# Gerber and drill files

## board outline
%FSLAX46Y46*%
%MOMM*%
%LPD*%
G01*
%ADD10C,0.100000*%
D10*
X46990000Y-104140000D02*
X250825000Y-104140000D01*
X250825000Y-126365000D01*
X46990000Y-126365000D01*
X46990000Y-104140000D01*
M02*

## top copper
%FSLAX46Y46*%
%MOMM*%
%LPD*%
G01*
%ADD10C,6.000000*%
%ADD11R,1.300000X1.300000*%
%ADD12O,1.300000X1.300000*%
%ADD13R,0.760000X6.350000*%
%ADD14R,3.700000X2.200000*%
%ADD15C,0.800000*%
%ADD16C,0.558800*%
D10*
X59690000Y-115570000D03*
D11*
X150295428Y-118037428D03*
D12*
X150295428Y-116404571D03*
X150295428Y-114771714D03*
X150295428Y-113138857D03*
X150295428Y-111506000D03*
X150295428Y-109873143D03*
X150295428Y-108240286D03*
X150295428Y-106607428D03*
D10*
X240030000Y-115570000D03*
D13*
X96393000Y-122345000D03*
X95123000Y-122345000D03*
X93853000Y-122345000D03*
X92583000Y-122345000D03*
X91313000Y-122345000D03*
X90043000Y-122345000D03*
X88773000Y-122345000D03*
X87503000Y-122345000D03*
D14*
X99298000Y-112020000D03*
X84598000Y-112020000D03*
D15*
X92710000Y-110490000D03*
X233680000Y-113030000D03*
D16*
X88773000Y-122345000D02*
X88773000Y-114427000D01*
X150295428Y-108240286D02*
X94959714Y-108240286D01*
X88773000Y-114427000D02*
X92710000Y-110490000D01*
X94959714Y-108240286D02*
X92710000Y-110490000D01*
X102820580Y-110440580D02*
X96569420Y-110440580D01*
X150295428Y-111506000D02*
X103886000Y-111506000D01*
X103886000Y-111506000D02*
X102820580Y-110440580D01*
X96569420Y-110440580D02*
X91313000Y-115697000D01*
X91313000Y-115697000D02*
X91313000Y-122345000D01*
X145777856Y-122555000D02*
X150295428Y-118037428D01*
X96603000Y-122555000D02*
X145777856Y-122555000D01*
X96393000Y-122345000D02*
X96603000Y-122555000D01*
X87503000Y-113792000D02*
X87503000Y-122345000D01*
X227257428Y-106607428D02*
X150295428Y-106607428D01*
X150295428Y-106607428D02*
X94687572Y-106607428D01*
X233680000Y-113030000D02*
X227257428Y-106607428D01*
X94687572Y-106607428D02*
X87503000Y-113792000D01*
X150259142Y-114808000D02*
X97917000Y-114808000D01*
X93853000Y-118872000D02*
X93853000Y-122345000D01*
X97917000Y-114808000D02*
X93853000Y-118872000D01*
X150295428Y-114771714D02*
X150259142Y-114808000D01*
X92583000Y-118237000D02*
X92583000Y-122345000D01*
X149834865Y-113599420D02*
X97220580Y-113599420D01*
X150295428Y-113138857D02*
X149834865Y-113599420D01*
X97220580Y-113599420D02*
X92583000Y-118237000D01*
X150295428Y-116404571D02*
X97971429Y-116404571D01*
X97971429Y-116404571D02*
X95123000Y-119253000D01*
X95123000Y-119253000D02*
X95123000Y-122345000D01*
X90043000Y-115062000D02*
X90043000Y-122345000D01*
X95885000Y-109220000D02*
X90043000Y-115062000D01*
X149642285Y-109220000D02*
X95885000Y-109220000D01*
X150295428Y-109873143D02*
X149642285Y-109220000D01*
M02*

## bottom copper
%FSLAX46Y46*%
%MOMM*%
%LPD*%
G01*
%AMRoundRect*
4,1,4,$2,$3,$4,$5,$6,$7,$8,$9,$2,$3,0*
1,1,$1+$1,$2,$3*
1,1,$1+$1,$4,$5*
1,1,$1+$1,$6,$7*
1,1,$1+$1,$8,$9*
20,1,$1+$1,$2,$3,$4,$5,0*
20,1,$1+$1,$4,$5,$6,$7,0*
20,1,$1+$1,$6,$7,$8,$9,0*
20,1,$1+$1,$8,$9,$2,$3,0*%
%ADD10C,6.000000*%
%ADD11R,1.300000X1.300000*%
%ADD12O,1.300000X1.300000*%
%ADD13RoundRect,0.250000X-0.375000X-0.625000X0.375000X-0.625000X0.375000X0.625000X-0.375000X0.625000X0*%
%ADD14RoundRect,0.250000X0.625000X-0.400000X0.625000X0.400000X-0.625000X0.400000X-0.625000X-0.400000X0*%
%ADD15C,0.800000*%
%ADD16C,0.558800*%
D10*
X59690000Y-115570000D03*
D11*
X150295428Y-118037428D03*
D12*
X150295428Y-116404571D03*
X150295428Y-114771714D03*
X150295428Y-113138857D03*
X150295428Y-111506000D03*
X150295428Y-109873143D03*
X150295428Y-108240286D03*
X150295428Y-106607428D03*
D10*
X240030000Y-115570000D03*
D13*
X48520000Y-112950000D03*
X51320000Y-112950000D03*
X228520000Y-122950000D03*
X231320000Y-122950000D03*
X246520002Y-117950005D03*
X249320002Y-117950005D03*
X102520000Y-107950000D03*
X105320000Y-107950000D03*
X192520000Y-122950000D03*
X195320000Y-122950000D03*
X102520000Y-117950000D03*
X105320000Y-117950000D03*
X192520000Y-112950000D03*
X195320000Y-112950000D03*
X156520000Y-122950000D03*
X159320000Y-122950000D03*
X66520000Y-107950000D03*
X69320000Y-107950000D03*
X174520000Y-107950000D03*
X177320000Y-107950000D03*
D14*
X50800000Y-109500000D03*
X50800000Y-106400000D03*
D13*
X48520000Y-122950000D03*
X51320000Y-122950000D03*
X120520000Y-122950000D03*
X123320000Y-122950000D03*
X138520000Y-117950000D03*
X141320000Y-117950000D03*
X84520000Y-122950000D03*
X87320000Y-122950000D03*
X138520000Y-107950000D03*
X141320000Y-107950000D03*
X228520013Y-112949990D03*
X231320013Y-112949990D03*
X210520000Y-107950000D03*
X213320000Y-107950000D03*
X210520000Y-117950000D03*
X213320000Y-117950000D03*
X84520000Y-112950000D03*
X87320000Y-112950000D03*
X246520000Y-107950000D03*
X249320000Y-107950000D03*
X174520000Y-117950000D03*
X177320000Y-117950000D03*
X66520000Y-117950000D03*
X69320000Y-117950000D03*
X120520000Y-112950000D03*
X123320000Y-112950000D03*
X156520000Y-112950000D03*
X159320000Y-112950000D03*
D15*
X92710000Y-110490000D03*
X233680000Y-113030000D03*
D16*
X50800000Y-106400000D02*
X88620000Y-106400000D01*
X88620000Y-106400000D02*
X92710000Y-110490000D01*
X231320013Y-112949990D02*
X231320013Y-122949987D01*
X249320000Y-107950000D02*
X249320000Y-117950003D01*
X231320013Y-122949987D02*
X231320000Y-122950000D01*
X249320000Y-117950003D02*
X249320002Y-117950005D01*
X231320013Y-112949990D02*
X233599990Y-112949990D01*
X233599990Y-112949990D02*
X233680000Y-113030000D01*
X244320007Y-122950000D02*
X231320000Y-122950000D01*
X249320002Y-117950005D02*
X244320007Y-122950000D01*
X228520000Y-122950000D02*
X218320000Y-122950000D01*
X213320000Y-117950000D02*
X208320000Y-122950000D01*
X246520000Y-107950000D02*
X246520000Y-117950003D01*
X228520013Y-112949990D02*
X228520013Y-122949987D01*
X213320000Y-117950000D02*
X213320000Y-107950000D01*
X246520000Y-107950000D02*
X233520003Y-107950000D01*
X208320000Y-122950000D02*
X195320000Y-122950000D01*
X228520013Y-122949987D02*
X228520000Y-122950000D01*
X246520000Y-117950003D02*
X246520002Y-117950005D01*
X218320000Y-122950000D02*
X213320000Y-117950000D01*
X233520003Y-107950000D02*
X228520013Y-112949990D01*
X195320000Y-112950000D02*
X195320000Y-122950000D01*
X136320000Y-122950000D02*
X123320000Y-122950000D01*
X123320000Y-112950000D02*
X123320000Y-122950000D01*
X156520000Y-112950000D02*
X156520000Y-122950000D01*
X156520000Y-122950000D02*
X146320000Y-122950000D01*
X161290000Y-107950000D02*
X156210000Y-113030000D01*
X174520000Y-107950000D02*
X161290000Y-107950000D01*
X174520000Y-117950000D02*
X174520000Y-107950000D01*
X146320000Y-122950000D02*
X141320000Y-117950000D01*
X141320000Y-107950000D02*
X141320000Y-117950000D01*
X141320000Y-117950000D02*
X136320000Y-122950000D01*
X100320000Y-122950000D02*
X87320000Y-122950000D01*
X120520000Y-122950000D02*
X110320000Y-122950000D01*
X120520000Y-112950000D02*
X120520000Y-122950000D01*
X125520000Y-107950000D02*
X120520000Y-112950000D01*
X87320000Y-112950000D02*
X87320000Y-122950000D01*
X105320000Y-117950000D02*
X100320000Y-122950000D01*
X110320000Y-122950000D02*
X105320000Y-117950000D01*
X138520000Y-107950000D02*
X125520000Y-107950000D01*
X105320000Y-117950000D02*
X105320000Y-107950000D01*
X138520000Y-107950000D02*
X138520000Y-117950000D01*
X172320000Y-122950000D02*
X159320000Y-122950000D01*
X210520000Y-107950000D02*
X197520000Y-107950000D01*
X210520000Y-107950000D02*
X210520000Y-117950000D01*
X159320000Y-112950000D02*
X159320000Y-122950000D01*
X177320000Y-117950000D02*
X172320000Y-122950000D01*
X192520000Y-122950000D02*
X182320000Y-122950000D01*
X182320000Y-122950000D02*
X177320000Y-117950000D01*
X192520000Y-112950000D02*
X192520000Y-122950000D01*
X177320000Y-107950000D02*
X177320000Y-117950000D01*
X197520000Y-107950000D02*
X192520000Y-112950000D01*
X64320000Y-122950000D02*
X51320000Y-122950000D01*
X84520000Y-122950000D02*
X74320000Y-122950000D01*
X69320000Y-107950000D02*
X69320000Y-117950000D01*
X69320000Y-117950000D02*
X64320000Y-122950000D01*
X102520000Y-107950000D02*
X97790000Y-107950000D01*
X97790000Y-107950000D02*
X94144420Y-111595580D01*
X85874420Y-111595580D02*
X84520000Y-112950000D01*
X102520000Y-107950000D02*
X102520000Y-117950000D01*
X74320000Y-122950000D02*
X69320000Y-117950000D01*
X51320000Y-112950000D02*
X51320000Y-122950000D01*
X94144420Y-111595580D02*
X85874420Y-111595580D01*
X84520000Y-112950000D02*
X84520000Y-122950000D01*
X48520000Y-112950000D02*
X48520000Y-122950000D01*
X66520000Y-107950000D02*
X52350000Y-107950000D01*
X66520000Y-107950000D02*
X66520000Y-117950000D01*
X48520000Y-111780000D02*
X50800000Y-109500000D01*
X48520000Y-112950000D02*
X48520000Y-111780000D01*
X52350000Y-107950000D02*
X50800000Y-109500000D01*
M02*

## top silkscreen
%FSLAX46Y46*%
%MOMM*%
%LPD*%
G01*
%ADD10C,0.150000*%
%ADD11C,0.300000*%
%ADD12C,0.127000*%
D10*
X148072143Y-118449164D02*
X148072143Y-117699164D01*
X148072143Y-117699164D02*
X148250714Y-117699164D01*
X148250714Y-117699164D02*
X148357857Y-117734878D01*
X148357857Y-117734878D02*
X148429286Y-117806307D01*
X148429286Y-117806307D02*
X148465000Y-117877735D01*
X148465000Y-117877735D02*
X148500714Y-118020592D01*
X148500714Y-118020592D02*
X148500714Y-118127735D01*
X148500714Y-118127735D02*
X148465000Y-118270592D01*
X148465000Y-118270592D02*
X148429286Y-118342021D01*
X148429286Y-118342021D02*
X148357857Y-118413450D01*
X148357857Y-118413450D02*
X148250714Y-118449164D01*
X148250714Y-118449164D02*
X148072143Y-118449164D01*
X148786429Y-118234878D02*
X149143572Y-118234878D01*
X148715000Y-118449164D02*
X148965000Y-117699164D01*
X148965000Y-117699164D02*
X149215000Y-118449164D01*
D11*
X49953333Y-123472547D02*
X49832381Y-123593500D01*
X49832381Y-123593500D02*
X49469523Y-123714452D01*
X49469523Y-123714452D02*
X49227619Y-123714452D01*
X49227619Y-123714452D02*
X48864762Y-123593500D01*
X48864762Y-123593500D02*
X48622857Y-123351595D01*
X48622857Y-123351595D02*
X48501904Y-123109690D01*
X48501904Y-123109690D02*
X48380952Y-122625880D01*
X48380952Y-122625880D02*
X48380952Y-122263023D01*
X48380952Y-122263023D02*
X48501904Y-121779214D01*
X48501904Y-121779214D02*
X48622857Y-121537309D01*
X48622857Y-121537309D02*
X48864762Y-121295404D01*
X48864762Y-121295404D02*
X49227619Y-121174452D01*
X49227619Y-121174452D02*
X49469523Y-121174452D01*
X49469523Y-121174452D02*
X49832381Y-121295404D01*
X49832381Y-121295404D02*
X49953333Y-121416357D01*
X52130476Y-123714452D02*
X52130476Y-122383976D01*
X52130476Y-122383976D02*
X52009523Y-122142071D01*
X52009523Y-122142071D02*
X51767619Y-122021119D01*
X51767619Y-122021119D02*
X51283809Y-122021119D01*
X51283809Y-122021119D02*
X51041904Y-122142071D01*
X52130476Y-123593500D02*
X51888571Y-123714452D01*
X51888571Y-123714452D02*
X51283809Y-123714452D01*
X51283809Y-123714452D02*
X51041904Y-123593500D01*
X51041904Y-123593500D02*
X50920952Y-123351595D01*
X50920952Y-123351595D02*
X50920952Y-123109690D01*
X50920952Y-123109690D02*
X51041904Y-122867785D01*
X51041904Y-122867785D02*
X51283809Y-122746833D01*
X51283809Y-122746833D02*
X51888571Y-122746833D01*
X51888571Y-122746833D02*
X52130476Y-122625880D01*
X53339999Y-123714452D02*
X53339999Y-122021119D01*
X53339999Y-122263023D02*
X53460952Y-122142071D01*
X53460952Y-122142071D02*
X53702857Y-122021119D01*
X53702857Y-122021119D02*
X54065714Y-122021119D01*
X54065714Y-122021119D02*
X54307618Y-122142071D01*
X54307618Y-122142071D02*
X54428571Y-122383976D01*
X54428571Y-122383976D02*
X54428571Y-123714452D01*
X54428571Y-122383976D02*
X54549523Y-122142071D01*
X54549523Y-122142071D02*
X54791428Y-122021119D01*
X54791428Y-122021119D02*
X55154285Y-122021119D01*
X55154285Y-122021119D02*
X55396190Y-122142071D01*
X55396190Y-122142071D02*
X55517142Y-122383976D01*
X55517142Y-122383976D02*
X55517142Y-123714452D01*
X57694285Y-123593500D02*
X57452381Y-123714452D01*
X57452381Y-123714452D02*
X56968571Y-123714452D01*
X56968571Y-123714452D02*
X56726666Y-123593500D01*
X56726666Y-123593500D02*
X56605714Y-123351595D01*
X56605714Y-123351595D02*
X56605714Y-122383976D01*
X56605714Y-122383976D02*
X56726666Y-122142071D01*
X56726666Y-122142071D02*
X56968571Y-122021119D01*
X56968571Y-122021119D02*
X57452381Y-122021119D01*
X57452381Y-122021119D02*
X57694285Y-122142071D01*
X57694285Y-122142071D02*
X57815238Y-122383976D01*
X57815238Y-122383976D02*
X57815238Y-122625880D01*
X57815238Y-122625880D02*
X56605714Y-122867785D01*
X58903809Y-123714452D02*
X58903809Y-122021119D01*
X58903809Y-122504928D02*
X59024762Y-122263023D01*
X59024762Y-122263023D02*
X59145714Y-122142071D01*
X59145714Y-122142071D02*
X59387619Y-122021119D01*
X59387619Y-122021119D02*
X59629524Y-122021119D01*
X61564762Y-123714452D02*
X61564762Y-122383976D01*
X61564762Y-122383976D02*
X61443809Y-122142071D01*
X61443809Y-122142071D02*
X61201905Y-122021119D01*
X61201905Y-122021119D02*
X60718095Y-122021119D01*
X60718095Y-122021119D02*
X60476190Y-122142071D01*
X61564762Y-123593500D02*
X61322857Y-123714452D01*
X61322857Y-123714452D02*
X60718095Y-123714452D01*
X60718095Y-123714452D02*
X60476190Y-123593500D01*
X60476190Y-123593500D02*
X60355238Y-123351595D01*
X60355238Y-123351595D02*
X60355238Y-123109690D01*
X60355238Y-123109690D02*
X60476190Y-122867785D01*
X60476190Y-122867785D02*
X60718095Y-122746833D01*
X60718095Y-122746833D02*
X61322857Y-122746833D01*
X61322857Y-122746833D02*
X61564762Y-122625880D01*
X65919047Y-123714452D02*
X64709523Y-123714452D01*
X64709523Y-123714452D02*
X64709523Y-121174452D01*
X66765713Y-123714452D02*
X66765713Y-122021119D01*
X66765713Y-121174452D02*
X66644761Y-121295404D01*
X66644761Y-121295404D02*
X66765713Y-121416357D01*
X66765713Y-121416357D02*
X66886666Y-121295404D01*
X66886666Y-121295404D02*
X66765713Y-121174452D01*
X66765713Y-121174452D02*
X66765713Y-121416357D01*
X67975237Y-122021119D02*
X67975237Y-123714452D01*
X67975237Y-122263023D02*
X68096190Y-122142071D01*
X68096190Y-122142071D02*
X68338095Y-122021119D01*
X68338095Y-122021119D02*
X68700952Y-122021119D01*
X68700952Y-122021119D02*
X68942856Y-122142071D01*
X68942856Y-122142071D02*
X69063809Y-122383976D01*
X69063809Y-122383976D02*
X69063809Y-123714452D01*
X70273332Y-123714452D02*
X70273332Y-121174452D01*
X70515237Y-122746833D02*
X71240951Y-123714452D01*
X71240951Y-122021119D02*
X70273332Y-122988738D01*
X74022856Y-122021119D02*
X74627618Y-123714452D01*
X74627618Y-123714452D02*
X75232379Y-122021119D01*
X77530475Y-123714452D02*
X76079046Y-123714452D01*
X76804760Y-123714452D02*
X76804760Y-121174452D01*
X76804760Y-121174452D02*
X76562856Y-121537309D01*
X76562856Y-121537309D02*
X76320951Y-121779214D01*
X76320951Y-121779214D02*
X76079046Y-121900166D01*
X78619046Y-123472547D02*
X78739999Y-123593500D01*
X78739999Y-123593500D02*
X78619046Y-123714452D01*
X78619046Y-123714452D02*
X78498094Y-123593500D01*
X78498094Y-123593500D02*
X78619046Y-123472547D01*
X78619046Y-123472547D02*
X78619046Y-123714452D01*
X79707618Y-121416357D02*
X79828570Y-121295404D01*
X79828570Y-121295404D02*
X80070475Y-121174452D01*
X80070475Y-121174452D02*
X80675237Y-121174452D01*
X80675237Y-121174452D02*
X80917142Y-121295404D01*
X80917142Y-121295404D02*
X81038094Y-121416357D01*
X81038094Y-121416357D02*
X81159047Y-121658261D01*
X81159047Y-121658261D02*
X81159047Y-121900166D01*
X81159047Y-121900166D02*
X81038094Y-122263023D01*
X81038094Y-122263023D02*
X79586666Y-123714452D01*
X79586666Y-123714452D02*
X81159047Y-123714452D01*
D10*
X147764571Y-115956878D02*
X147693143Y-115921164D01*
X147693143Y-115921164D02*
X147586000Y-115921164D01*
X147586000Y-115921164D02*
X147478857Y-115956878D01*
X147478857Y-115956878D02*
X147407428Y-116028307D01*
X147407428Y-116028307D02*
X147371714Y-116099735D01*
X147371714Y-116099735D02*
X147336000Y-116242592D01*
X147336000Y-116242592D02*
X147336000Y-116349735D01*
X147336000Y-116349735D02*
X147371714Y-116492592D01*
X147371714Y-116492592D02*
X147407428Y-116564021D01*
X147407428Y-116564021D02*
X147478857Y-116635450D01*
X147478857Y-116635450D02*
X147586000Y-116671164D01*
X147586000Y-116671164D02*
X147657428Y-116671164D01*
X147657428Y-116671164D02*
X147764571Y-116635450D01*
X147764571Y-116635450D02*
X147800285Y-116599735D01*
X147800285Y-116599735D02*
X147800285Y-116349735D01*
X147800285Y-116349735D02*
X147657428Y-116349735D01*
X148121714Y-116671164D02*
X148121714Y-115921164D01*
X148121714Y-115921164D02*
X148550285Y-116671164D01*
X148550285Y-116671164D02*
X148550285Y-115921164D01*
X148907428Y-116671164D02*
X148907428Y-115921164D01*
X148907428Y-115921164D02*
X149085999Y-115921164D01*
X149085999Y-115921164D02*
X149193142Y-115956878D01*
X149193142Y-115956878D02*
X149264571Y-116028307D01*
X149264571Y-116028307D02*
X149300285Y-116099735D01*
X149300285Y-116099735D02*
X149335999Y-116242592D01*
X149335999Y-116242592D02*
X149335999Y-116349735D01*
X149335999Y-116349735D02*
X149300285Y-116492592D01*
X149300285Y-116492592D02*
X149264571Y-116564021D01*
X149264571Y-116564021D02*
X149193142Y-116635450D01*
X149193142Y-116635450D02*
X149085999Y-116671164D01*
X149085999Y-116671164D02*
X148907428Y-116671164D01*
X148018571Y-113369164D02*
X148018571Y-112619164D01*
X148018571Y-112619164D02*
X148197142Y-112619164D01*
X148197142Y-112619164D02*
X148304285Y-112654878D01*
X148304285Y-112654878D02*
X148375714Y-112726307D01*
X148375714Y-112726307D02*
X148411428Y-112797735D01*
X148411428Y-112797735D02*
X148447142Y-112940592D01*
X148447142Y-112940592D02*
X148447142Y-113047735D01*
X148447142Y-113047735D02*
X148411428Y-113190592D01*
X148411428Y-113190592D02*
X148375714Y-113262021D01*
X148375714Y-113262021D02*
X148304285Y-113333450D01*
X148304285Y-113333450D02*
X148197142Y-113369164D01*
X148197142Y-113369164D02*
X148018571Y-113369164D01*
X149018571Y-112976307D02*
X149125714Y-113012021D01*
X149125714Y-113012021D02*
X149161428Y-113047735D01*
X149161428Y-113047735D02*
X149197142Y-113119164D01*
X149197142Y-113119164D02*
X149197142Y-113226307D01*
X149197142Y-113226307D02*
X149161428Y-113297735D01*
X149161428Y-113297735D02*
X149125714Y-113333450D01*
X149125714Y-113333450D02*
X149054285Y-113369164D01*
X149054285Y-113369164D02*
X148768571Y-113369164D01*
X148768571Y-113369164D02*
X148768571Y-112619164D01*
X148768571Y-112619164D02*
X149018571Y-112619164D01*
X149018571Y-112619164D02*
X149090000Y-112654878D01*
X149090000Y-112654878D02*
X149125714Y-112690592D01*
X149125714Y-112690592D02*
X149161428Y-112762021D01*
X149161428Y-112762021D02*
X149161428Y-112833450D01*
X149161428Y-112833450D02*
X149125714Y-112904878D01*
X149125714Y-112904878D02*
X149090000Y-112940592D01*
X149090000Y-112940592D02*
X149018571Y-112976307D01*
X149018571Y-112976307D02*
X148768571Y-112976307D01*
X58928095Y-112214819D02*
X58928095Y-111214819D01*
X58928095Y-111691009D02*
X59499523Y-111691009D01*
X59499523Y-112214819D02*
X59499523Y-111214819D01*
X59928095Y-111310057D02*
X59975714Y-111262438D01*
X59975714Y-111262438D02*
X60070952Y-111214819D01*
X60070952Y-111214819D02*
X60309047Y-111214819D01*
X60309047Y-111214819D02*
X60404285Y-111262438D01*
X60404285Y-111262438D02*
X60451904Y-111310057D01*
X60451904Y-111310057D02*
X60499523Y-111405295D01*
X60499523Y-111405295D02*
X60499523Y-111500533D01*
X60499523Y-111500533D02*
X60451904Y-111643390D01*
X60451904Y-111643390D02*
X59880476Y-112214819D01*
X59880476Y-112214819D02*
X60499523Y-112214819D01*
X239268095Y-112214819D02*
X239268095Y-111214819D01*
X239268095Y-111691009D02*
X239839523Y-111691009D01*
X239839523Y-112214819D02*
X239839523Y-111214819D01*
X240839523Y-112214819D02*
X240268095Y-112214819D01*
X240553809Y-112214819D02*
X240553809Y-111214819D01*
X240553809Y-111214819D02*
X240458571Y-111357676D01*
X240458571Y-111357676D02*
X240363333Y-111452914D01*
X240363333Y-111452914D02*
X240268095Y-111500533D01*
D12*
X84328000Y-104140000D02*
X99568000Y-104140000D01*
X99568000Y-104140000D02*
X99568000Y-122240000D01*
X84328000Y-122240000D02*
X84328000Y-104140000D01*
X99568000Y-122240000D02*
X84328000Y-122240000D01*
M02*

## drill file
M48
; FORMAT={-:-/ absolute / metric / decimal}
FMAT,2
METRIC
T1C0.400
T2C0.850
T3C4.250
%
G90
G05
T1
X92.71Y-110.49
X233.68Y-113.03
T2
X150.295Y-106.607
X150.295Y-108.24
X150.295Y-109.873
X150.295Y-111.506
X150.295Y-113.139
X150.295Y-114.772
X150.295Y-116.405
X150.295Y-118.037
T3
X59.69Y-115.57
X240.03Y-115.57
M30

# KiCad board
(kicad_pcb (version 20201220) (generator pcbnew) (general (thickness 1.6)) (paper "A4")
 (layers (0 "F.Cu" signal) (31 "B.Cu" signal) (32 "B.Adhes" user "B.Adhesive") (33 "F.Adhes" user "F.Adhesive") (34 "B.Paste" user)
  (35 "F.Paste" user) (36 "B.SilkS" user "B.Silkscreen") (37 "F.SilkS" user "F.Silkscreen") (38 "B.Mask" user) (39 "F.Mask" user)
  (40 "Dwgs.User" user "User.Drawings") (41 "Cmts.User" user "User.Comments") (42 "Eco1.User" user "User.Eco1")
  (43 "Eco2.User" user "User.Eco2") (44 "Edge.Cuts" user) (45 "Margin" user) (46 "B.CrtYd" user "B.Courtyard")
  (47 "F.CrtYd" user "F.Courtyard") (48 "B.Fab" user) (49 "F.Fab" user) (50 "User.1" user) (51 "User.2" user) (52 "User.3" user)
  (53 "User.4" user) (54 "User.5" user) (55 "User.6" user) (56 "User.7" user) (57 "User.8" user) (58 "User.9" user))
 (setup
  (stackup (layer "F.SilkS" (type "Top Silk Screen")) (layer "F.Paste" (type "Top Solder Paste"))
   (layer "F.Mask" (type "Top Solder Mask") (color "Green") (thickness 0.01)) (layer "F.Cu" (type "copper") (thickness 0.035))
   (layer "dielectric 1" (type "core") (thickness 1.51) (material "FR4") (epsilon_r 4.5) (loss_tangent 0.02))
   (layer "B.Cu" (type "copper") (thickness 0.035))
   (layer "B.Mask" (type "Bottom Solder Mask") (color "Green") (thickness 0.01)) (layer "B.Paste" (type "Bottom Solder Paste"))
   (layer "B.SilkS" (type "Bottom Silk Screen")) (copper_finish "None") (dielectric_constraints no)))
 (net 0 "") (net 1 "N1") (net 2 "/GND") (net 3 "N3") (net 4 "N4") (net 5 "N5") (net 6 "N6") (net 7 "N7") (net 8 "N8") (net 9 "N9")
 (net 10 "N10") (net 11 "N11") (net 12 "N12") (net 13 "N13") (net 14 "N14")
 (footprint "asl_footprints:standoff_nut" (layer "F.Cu") (at 59.69 115.57)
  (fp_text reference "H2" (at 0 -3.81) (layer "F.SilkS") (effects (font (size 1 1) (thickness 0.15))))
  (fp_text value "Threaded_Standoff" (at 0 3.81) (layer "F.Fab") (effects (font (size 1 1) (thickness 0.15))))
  (pad "M3" thru_hole circle (at 0 0) (size 6 6) (drill 4.25) (layers *.Cu *.Mask)))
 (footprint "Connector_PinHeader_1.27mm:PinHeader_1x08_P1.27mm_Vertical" (layer "F.Cu") (at 150.295428 112.322429 180)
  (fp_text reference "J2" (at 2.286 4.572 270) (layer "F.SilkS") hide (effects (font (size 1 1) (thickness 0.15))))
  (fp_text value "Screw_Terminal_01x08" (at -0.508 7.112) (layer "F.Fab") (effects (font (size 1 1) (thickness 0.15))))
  (pad "1" thru_hole rect (at 0 -5.714999 180) (size 1.3 1.3) (drill 0.85) (layers *.Cu *.Mask) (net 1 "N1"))
  (pad "2" thru_hole oval (at 0 -4.082142 180) (size 1.3 1.3) (drill 0.85) (layers *.Cu *.Mask) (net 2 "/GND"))
  (pad "3" thru_hole oval (at 0 -2.449285 180) (size 1.3 1.3) (drill 0.85) (layers *.Cu *.Mask) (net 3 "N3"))
  (pad "4" thru_hole oval (at 0 -0.816428 180) (size 1.3 1.3) (drill 0.85) (layers *.Cu *.Mask) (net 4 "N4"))
  (pad "5" thru_hole oval (at 0 0.816429 180) (size 1.3 1.3) (drill 0.85) (layers *.Cu *.Mask) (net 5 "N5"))
  (pad "6" thru_hole oval (at 0 2.449286 180) (size 1.3 1.3) (drill 0.85) (layers *.Cu *.Mask) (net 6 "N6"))
  (pad "7" thru_hole oval (at 0 4.082143 180) (size 1.3 1.3) (drill 0.85) (layers *.Cu *.Mask) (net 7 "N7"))
  (pad "8" thru_hole oval (at 0 5.715001 180) (size 1.3 1.3) (drill 0.85) (layers *.Cu *.Mask) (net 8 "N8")))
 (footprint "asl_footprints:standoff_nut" (layer "F.Cu") (at 240.03 115.57)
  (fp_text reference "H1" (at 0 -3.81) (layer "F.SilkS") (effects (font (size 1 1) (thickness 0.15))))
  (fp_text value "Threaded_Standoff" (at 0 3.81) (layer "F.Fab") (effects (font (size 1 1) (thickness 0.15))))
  (pad "M3" thru_hole circle (at 0 0) (size 6 6) (drill 4.25) (layers *.Cu *.Mask)))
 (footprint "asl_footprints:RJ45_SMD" (layer "F.Cu") (at 91.948 104.14 180)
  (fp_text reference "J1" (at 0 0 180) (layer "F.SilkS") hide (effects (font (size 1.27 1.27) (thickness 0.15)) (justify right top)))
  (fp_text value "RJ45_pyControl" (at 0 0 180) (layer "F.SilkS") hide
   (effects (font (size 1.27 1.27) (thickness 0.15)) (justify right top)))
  (fp_line (start 7.62 0) (end -7.62 0) (layer "F.SilkS") (width 0.127))
  (fp_line (start -7.62 0) (end -7.62 -18.1) (layer "F.SilkS") (width 0.127))
  (fp_line (start 7.62 -18.1) (end 7.62 0) (layer "F.SilkS") (width 0.127))
  (fp_line (start -7.62 -18.1) (end 7.62 -18.1) (layer "F.SilkS") (width 0.127))
  (pad "1" smd rect (at -4.445 -18.205 270) (size 6.35 0.76) (layers "F.Cu" "F.Paste" "F.Mask") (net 1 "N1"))
  (pad "2" smd rect (at -3.175 -18.205 270) (size 6.35 0.76) (layers "F.Cu" "F.Paste" "F.Mask") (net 2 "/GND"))
  (pad "3" smd rect (at -1.905 -18.205 270) (size 6.35 0.76) (layers "F.Cu" "F.Paste" "F.Mask") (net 3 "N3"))
  (pad "4" smd rect (at -0.635 -18.205 270) (size 6.35 0.76) (layers "F.Cu" "F.Paste" "F.Mask") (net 4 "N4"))
  (pad "5" smd rect (at 0.635 -18.205 270) (size 6.35 0.76) (layers "F.Cu" "F.Paste" "F.Mask") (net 5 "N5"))
  (pad "6" smd rect (at 1.905 -18.205 270) (size 6.35 0.76) (layers "F.Cu" "F.Paste" "F.Mask") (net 6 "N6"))
  (pad "7" smd rect (at 3.175 -18.205 270) (size 6.35 0.76) (layers "F.Cu" "F.Paste" "F.Mask") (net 7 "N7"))
  (pad "8" smd rect (at 4.445 -18.205 270) (size 6.35 0.76) (layers "F.Cu" "F.Paste" "F.Mask") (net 8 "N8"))
  (pad "G1" smd rect (at -7.35 -7.88 180) (size 3.7 2.2) (layers "F.Cu" "F.Paste" "F.Mask"))
  (pad "G2" smd rect (at 7.35 -7.88 180) (size 3.7 2.2) (layers "F.Cu" "F.Paste" "F.Mask")))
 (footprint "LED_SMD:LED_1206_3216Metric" (layer "B.Cu") (at 49.92 112.95)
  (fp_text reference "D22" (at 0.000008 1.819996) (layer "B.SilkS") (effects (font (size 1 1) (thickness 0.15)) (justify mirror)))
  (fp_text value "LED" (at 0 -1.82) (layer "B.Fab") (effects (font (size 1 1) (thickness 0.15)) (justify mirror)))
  (pad "1" smd roundrect (at -1.4 0) (size 1.25 1.75) (layers "B.Cu" "B.Paste" "B.Mask") (roundrect_rratio 0.2) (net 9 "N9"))
  (pad "2" smd roundrect (at 1.4 0) (size 1.25 1.75) (layers "B.Cu" "B.Paste" "B.Mask") (roundrect_rratio 0.2) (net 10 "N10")))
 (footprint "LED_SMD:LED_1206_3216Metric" (layer "B.Cu") (at 229.92 122.95)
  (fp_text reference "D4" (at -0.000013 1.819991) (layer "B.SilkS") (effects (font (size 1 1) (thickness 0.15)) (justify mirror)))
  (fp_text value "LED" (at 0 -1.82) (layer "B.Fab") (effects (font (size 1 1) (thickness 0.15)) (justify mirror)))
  (pad "1" smd roundrect (at -1.4 0) (size 1.25 1.75) (layers "B.Cu" "B.Paste" "B.Mask") (roundrect_rratio 0.2) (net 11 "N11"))
  (pad "2" smd roundrect (at 1.4 0) (size 1.25 1.75) (layers "B.Cu" "B.Paste" "B.Mask") (roundrect_rratio 0.2) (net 8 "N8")))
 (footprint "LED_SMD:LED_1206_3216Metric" (layer "B.Cu") (at 247.920002 117.950005)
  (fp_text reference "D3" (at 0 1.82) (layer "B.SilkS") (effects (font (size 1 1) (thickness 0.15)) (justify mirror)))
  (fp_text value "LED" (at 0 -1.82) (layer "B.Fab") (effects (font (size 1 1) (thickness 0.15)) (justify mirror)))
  (pad "1" smd roundrect (at -1.4 0) (size 1.25 1.75) (layers "B.Cu" "B.Paste" "B.Mask") (roundrect_rratio 0.2) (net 11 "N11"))
  (pad "2" smd roundrect (at 1.4 0) (size 1.25 1.75) (layers "B.Cu" "B.Paste" "B.Mask") (roundrect_rratio 0.2) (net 8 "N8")))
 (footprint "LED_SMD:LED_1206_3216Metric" (layer "B.Cu") (at 103.92 107.95)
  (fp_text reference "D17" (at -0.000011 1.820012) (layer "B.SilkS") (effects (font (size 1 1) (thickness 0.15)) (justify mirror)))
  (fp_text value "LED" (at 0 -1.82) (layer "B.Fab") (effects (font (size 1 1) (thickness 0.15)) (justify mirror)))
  (pad "1" smd roundrect (at -1.4 0) (size 1.25 1.75) (layers "B.Cu" "B.Paste" "B.Mask") (roundrect_rratio 0.2) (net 10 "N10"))
  (pad "2" smd roundrect (at 1.4 0) (size 1.25 1.75) (layers "B.Cu" "B.Paste" "B.Mask") (roundrect_rratio 0.2) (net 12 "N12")))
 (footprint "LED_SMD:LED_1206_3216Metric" (layer "B.Cu") (at 193.92 122.95)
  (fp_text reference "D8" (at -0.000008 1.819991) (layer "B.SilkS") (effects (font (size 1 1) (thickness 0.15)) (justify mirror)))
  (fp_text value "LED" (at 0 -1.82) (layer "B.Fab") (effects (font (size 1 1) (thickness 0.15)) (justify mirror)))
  (pad "1" smd roundrect (at -1.4 0) (size 1.25 1.75) (layers "B.Cu" "B.Paste" "B.Mask") (roundrect_rratio 0.2) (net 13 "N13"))
  (pad "2" smd roundrect (at 1.4 0) (size 1.25 1.75) (layers "B.Cu" "B.Paste" "B.Mask") (roundrect_rratio 0.2) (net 11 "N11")))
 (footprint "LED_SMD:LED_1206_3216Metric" (layer "B.Cu") (at 103.92 117.95)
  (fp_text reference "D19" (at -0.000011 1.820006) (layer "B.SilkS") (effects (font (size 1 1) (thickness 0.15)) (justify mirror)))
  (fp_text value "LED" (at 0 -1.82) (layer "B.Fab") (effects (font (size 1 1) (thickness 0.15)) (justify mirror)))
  (pad "1" smd roundrect (at -1.4 0) (size 1.25 1.75) (layers "B.Cu" "B.Paste" "B.Mask") (roundrect_rratio 0.2) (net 10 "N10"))
  (pad "2" smd roundrect (at 1.4 0) (size 1.25 1.75) (layers "B.Cu" "B.Paste" "B.Mask") (roundrect_rratio 0.2) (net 12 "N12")))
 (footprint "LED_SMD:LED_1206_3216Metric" (layer "B.Cu") (at 193.92 112.95)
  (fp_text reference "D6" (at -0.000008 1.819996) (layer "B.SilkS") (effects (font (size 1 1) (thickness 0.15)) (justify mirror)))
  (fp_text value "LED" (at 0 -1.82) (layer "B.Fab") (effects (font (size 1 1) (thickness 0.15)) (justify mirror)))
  (pad "1" smd roundrect (at -1.4 0) (size 1.25 1.75) (layers "B.Cu" "B.Paste" "B.Mask") (roundrect_rratio 0.2) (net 13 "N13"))
  (pad "2" smd roundrect (at 1.4 0) (size 1.25 1.75) (layers "B.Cu" "B.Paste" "B.Mask") (roundrect_rratio 0.2) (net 11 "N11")))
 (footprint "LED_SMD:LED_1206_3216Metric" (layer "B.Cu") (at 157.92 122.95)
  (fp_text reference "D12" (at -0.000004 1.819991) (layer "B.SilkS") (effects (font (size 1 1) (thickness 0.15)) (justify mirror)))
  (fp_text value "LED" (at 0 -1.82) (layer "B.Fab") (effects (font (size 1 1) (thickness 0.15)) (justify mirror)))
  (pad "1" smd roundrect (at -1.4 0) (size 1.25 1.75) (layers "B.Cu" "B.Paste" "B.Mask") (roundrect_rratio 0.2) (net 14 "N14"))
  (pad "2" smd roundrect (at 1.4 0) (size 1.25 1.75) (layers "B.Cu" "B.Paste" "B.Mask") (roundrect_rratio 0.2) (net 13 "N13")))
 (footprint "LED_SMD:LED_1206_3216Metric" (layer "B.Cu") (at 67.92 107.95)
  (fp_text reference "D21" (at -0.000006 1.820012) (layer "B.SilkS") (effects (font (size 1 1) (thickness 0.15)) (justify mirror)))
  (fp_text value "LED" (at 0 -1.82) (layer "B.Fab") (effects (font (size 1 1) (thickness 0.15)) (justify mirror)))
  (pad "1" smd roundrect (at -1.4 0) (size 1.25 1.75) (layers "B.Cu" "B.Paste" "B.Mask") (roundrect_rratio 0.2) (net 9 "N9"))
  (pad "2" smd roundrect (at 1.4 0) (size 1.25 1.75) (layers "B.Cu" "B.Paste" "B.Mask") (roundrect_rratio 0.2) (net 10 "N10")))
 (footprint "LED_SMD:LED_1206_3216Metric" (layer "B.Cu") (at 175.92 107.95)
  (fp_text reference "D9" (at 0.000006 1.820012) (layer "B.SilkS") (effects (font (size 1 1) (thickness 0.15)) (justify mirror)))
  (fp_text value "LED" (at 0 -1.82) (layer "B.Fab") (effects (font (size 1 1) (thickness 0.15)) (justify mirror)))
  (pad "1" smd roundrect (at -1.4 0) (size 1.25 1.75) (layers "B.Cu" "B.Paste" "B.Mask") (roundrect_rratio 0.2) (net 14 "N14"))
  (pad "2" smd roundrect (at 1.4 0) (size 1.25 1.75) (layers "B.Cu" "B.Paste" "B.Mask") (roundrect_rratio 0.2) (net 13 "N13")))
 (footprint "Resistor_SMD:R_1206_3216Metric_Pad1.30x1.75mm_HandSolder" (layer "B.Cu") (at 50.8 107.95 90)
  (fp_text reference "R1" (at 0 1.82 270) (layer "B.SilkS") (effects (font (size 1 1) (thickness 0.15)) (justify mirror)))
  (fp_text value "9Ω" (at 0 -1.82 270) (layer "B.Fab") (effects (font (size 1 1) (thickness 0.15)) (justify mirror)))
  (pad "1" smd roundrect (at -1.55 0 90) (size 1.3 1.75) (layers "B.Cu" "B.Paste" "B.Mask") (roundrect_rratio 0.192308) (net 9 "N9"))
  (pad "2" smd roundrect (at 1.55 0 90) (size 1.3 1.75) (layers "B.Cu" "B.Paste" "B.Mask") (roundrect_rratio 0.192308) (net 7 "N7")))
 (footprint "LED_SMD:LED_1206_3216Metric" (layer "B.Cu") (at 49.92 122.95)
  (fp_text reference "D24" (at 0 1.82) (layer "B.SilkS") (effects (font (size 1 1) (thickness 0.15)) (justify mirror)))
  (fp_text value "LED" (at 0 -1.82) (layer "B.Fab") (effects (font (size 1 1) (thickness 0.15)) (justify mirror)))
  (pad "1" smd roundrect (at -1.4 0) (size 1.25 1.75) (layers "B.Cu" "B.Paste" "B.Mask") (roundrect_rratio 0.2) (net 9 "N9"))
  (pad "2" smd roundrect (at 1.4 0) (size 1.25 1.75) (layers "B.Cu" "B.Paste" "B.Mask") (roundrect_rratio 0.2) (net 10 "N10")))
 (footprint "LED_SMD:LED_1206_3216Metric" (layer "B.Cu") (at 121.92 122.95)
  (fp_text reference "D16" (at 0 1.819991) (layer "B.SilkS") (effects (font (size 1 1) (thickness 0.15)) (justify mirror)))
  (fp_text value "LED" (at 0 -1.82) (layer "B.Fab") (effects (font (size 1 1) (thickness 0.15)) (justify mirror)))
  (pad "1" smd roundrect (at -1.4 0) (size 1.25 1.75) (layers "B.Cu" "B.Paste" "B.Mask") (roundrect_rratio 0.2) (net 12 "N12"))
  (pad "2" smd roundrect (at 1.4 0) (size 1.25 1.75) (layers "B.Cu" "B.Paste" "B.Mask") (roundrect_rratio 0.2) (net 14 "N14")))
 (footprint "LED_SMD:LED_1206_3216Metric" (layer "B.Cu") (at 139.92 117.95)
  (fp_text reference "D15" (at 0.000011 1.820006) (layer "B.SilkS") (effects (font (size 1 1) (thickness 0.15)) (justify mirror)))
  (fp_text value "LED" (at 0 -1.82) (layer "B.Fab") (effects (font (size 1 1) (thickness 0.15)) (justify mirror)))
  (pad "1" smd roundrect (at -1.4 0) (size 1.25 1.75) (layers "B.Cu" "B.Paste" "B.Mask") (roundrect_rratio 0.2) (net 12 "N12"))
  (pad "2" smd roundrect (at 1.4 0) (size 1.25 1.75) (layers "B.Cu" "B.Paste" "B.Mask") (roundrect_rratio 0.2) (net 14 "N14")))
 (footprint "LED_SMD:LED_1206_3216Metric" (layer "B.Cu") (at 85.92 122.95)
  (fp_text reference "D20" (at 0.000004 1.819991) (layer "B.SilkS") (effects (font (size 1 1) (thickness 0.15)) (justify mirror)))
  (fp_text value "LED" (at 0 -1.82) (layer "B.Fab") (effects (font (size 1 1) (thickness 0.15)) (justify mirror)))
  (pad "1" smd roundrect (at -1.4 0) (size 1.25 1.75) (layers "B.Cu" "B.Paste" "B.Mask") (roundrect_rratio 0.2) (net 10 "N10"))
  (pad "2" smd roundrect (at 1.4 0) (size 1.25 1.75) (layers "B.Cu" "B.Paste" "B.Mask") (roundrect_rratio 0.2) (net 12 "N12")))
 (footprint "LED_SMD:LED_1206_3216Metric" (layer "B.Cu") (at 139.92 107.95)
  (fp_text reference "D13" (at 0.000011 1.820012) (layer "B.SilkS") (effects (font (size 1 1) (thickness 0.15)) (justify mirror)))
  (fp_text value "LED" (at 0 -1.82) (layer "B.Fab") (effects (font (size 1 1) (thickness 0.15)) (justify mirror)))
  (pad "1" smd roundrect (at -1.4 0) (size 1.25 1.75) (layers "B.Cu" "B.Paste" "B.Mask") (roundrect_rratio 0.2) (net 12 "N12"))
  (pad "2" smd roundrect (at 1.4 0) (size 1.25 1.75) (layers "B.Cu" "B.Paste" "B.Mask") (roundrect_rratio 0.2) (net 14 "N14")))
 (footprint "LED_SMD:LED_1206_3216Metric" (layer "B.Cu") (at 229.920013 112.94999)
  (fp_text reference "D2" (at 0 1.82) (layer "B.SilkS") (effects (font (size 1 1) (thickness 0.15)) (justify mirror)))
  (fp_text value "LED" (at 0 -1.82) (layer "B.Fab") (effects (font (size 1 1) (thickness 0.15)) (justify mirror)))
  (pad "1" smd roundrect (at -1.4 0) (size 1.25 1.75) (layers "B.Cu" "B.Paste" "B.Mask") (roundrect_rratio 0.2) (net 11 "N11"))
  (pad "2" smd roundrect (at 1.4 0) (size 1.25 1.75) (layers "B.Cu" "B.Paste" "B.Mask") (roundrect_rratio 0.2) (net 8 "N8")))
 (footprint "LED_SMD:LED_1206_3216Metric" (layer "B.Cu") (at 211.92 107.95)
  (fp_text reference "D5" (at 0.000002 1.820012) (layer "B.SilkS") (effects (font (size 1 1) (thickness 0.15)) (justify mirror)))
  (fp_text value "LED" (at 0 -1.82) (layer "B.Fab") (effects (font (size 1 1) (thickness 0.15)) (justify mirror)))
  (pad "1" smd roundrect (at -1.4 0) (size 1.25 1.75) (layers "B.Cu" "B.Paste" "B.Mask") (roundrect_rratio 0.2) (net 13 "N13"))
  (pad "2" smd roundrect (at 1.4 0) (size 1.25 1.75) (layers "B.Cu" "B.Paste" "B.Mask") (roundrect_rratio 0.2) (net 11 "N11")))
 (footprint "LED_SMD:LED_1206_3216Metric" (layer "B.Cu") (at 211.92 117.95)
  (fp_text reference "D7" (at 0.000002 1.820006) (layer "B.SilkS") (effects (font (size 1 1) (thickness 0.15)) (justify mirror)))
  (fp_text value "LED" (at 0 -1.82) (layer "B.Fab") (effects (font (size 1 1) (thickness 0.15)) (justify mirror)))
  (pad "1" smd roundrect (at -1.4 0) (size 1.25 1.75) (layers "B.Cu" "B.Paste" "B.Mask") (roundrect_rratio 0.2) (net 13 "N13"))
  (pad "2" smd roundrect (at 1.4 0) (size 1.25 1.75) (layers "B.Cu" "B.Paste" "B.Mask") (roundrect_rratio 0.2) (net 11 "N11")))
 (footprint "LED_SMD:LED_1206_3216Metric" (layer "B.Cu") (at 85.92 112.95)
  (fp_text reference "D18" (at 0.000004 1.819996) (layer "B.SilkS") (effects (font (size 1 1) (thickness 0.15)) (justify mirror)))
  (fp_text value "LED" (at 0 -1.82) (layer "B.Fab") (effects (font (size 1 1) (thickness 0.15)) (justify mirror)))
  (pad "1" smd roundrect (at -1.4 0) (size 1.25 1.75) (layers "B.Cu" "B.Paste" "B.Mask") (roundrect_rratio 0.2) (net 10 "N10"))
  (pad "2" smd roundrect (at 1.4 0) (size 1.25 1.75) (layers "B.Cu" "B.Paste" "B.Mask") (roundrect_rratio 0.2) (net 12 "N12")))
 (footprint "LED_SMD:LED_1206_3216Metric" (layer "B.Cu") (at 247.92 107.95)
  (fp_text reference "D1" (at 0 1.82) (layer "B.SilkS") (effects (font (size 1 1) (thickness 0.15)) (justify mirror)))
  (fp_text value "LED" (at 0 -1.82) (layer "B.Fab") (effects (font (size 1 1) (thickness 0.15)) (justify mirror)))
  (pad "1" smd roundrect (at -1.4 0) (size 1.25 1.75) (layers "B.Cu" "B.Paste" "B.Mask") (roundrect_rratio 0.2) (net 11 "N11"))
  (pad "2" smd roundrect (at 1.4 0) (size 1.25 1.75) (layers "B.Cu" "B.Paste" "B.Mask") (roundrect_rratio 0.2) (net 8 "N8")))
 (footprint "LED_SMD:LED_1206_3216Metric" (layer "B.Cu") (at 175.92 117.95)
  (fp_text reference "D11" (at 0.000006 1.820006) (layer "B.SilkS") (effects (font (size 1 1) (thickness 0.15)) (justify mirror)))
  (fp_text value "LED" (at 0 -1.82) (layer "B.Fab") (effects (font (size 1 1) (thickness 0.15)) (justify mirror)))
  (pad "1" smd roundrect (at -1.4 0) (size 1.25 1.75) (layers "B.Cu" "B.Paste" "B.Mask") (roundrect_rratio 0.2) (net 14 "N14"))
  (pad "2" smd roundrect (at 1.4 0) (size 1.25 1.75) (layers "B.Cu" "B.Paste" "B.Mask") (roundrect_rratio 0.2) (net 13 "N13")))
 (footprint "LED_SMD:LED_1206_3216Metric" (layer "B.Cu") (at 67.92 117.95)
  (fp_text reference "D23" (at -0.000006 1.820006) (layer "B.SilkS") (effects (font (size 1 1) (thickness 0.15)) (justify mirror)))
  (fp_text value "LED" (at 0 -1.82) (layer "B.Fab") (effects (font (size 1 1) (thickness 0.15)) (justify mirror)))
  (pad "1" smd roundrect (at -1.4 0) (size 1.25 1.75) (layers "B.Cu" "B.Paste" "B.Mask") (roundrect_rratio 0.2) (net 9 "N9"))
  (pad "2" smd roundrect (at 1.4 0) (size 1.25 1.75) (layers "B.Cu" "B.Paste" "B.Mask") (roundrect_rratio 0.2) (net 10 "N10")))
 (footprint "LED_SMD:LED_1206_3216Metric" (layer "B.Cu") (at 121.92 112.95)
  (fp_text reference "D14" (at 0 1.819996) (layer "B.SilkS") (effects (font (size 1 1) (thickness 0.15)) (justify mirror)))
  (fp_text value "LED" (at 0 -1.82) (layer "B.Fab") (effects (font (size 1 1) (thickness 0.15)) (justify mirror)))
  (pad "1" smd roundrect (at -1.4 0) (size 1.25 1.75) (layers "B.Cu" "B.Paste" "B.Mask") (roundrect_rratio 0.2) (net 12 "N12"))
  (pad "2" smd roundrect (at 1.4 0) (size 1.25 1.75) (layers "B.Cu" "B.Paste" "B.Mask") (roundrect_rratio 0.2) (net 14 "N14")))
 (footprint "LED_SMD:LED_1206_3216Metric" (layer "B.Cu") (at 157.92 112.95)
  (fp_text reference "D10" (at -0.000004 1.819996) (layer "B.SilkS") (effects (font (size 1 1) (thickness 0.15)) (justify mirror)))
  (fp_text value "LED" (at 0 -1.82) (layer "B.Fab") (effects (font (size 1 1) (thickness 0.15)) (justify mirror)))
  (pad "1" smd roundrect (at -1.4 0) (size 1.25 1.75) (layers "B.Cu" "B.Paste" "B.Mask") (roundrect_rratio 0.2) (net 14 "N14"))
  (pad "2" smd roundrect (at 1.4 0) (size 1.25 1.75) (layers "B.Cu" "B.Paste" "B.Mask") (roundrect_rratio 0.2) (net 13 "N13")))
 (gr_rect (start 46.99 104.14) (end 250.825 126.365) (layer "Edge.Cuts") (width 0.1) (fill none))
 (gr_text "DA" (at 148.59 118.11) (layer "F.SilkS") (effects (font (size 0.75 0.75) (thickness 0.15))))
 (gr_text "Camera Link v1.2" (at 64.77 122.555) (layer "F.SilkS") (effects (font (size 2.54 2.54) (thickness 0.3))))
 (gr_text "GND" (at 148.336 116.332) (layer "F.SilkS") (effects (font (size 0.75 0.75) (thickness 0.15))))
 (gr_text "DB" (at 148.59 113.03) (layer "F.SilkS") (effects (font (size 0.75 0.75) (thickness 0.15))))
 (segment (start 88.773 122.345) (end 88.773 114.427) (width 0.5588) (layer "F.Cu") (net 7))
 (segment (start 150.295428 108.240286) (end 94.959714 108.240286) (width 0.5588) (layer "F.Cu") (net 7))
 (segment (start 88.773 114.427) (end 92.71 110.49) (width 0.5588) (layer "F.Cu") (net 7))
 (segment (start 94.959714 108.240286) (end 92.71 110.49) (width 0.5588) (layer "F.Cu") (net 7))
 (via (at 92.71 110.49) (size 0.8) (drill 0.4) (layers "F.Cu" "B.Cu") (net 7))
 (segment (start 50.8 106.4) (end 88.62 106.4) (width 0.5588) (layer "B.Cu") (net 7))
 (segment (start 88.62 106.4) (end 92.71 110.49) (width 0.5588) (layer "B.Cu") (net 7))
 (segment (start 102.82058 110.44058) (end 96.56942 110.44058) (width 0.5588) (layer "F.Cu") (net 5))
 (segment (start 150.295428 111.506) (end 103.886 111.506) (width 0.5588) (layer "F.Cu") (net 5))
 (segment (start 103.886 111.506) (end 102.82058 110.44058) (width 0.5588) (layer "F.Cu") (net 5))
 (segment (start 96.56942 110.44058) (end 91.313 115.697) (width 0.5588) (layer "F.Cu") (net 5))
 (segment (start 91.313 115.697) (end 91.313 122.345) (width 0.5588) (layer "F.Cu") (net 5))
 (segment (start 145.777856 122.555) (end 150.295428 118.037428) (width 0.5588) (layer "F.Cu") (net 1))
 (segment (start 96.603 122.555) (end 145.777856 122.555) (width 0.5588) (layer "F.Cu") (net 1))
 (segment (start 96.393 122.345) (end 96.603 122.555) (width 0.5588) (layer "F.Cu") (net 1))
 (segment (start 87.503 113.792) (end 87.503 122.345) (width 0.5588) (layer "F.Cu") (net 8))
 (segment (start 227.257428 106.607428) (end 150.295428 106.607428) (width 0.5588) (layer "F.Cu") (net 8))
 (segment (start 150.295428 106.607428) (end 94.687572 106.607428) (width 0.5588) (layer "F.Cu") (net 8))
 (segment (start 233.68 113.03) (end 227.257428 106.607428) (width 0.5588) (layer "F.Cu") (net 8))
 (segment (start 94.687572 106.607428) (end 87.503 113.792) (width 0.5588) (layer "F.Cu") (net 8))
 (via (at 233.68 113.03) (size 0.8) (drill 0.4) (layers "F.Cu" "B.Cu") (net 8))
 (segment (start 231.320013 112.94999) (end 231.320013 122.949987) (width 0.5588) (layer "B.Cu") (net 8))
 (segment (start 249.32 107.95) (end 249.32 117.950003) (width 0.5588) (layer "B.Cu") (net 8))
 (segment (start 231.320013 122.949987) (end 231.32 122.95) (width 0.5588) (layer "B.Cu") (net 8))
 (segment (start 249.32 117.950003) (end 249.320002 117.950005) (width 0.5588) (layer "B.Cu") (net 8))
 (segment (start 231.320013 112.94999) (end 233.59999 112.94999) (width 0.5588) (layer "B.Cu") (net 8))
 (segment (start 233.59999 112.94999) (end 233.68 113.03) (width 0.5588) (layer "B.Cu") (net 8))
 (segment (start 244.320007 122.95) (end 231.32 122.95) (width 0.5588) (layer "B.Cu") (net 8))
 (segment (start 249.320002 117.950005) (end 244.320007 122.95) (width 0.5588) (layer "B.Cu") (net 8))
 (segment (start 150.259142 114.808) (end 97.917 114.808) (width 0.5588) (layer "F.Cu") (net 3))
 (segment (start 93.853 118.872) (end 93.853 122.345) (width 0.5588) (layer "F.Cu") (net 3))
 (segment (start 97.917 114.808) (end 93.853 118.872) (width 0.5588) (layer "F.Cu") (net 3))
 (segment (start 150.295428 114.771714) (end 150.259142 114.808) (width 0.5588) (layer "F.Cu") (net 3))
 (segment (start 92.583 118.237) (end 92.583 122.345) (width 0.5588) (layer "F.Cu") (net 4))
 (segment (start 149.834865 113.59942) (end 97.22058 113.59942) (width 0.5588) (layer "F.Cu") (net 4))
 (segment (start 150.295428 113.138857) (end 149.834865 113.59942) (width 0.5588) (layer "F.Cu") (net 4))
 (segment (start 97.22058 113.59942) (end 92.583 118.237) (width 0.5588) (layer "F.Cu") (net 4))
 (segment (start 228.52 122.95) (end 218.32 122.95) (width 0.5588) (layer "B.Cu") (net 11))
 (segment (start 213.32 117.95) (end 208.32 122.95) (width 0.5588) (layer "B.Cu") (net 11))
 (segment (start 246.52 107.95) (end 246.52 117.950003) (width 0.5588) (layer "B.Cu") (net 11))
 (segment (start 228.520013 112.94999) (end 228.520013 122.949987) (width 0.5588) (layer "B.Cu") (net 11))
 (segment (start 213.32 117.95) (end 213.32 107.95) (width 0.5588) (layer "B.Cu") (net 11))
 (segment (start 246.52 107.95) (end 233.520003 107.95) (width 0.5588) (layer "B.Cu") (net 11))
 (segment (start 208.32 122.95) (end 195.32 122.95) (width 0.5588) (layer "B.Cu") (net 11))
 (segment (start 228.520013 122.949987) (end 228.52 122.95) (width 0.5588) (layer "B.Cu") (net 11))
 (segment (start 246.52 117.950003) (end 246.520002 117.950005) (width 0.5588) (layer "B.Cu") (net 11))
 (segment (start 218.32 122.95) (end 213.32 117.95) (width 0.5588) (layer "B.Cu") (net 11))
 (segment (start 233.520003 107.95) (end 228.520013 112.94999) (width 0.5588) (layer "B.Cu") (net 11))
 (segment (start 195.32 112.95) (end 195.32 122.95) (width 0.5588) (layer "B.Cu") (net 11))
 (segment (start 136.32 122.95) (end 123.32 122.95) (width 0.5588) (layer "B.Cu") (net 14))
 (segment (start 123.32 112.95) (end 123.32 122.95) (width 0.5588) (layer "B.Cu") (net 14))
 (segment (start 156.52 112.95) (end 156.52 122.95) (width 0.5588) (layer "B.Cu") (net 14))
 (segment (start 156.52 122.95) (end 146.32 122.95) (width 0.5588) (layer "B.Cu") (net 14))
 (segment (start 161.29 107.95) (end 156.21 113.03) (width 0.5588) (layer "B.Cu") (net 14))
 (segment (start 174.52 107.95) (end 161.29 107.95) (width 0.5588) (layer "B.Cu") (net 14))
 (segment (start 174.52 117.95) (end 174.52 107.95) (width 0.5588) (layer "B.Cu") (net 14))
 (segment (start 146.32 122.95) (end 141.32 117.95) (width 0.5588) (layer "B.Cu") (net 14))
 (segment (start 141.32 107.95) (end 141.32 117.95) (width 0.5588) (layer "B.Cu") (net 14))
 (segment (start 141.32 117.95) (end 136.32 122.95) (width 0.5588) (layer "B.Cu") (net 14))
 (segment (start 100.32 122.95) (end 87.32 122.95) (width 0.5588) (layer "B.Cu") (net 12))
 (segment (start 120.52 122.95) (end 110.32 122.95) (width 0.5588) (layer "B.Cu") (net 12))
 (segment (start 120.52 112.95) (end 120.52 122.95) (width 0.5588) (layer "B.Cu") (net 12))
 (segment (start 125.52 107.95) (end 120.52 112.95) (width 0.5588) (layer "B.Cu") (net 12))
 (segment (start 87.32 112.95) (end 87.32 122.95) (width 0.5588) (layer "B.Cu") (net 12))
 (segment (start 105.32 117.95) (end 100.32 122.95) (width 0.5588) (layer "B.Cu") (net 12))
 (segment (start 110.32 122.95) (end 105.32 117.95) (width 0.5588) (layer "B.Cu") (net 12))
 (segment (start 138.52 107.95) (end 125.52 107.95) (width 0.5588) (layer "B.Cu") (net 12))
 (segment (start 105.32 117.95) (end 105.32 107.95) (width 0.5588) (layer "B.Cu") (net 12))
 (segment (start 138.52 107.95) (end 138.52 117.95) (width 0.5588) (layer "B.Cu") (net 12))
 (segment (start 172.32 122.95) (end 159.32 122.95) (width 0.5588) (layer "B.Cu") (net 13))
 (segment (start 210.52 107.95) (end 197.52 107.95) (width 0.5588) (layer "B.Cu") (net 13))
 (segment (start 210.52 107.95) (end 210.52 117.95) (width 0.5588) (layer "B.Cu") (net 13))
 (segment (start 159.32 112.95) (end 159.32 122.95) (width 0.5588) (layer "B.Cu") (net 13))
 (segment (start 177.32 117.95) (end 172.32 122.95) (width 0.5588) (layer "B.Cu") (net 13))
 (segment (start 192.52 122.95) (end 182.32 122.95) (width 0.5588) (layer "B.Cu") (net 13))
 (segment (start 182.32 122.95) (end 177.32 117.95) (width 0.5588) (layer "B.Cu") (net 13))
 (segment (start 192.52 112.95) (end 192.52 122.95) (width 0.5588) (layer "B.Cu") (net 13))
 (segment (start 177.32 107.95) (end 177.32 117.95) (width 0.5588) (layer "B.Cu") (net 13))
 (segment (start 197.52 107.95) (end 192.52 112.95) (width 0.5588) (layer "B.Cu") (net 13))
 (segment (start 64.32 122.95) (end 51.32 122.95) (width 0.5588) (layer "B.Cu") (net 10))
 (segment (start 84.52 122.95) (end 74.32 122.95) (width 0.5588) (layer "B.Cu") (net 10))
 (segment (start 69.32 107.95) (end 69.32 117.95) (width 0.5588) (layer "B.Cu") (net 10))
 (segment (start 69.32 117.95) (end 64.32 122.95) (width 0.5588) (layer "B.Cu") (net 10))
 (segment (start 102.52 107.95) (end 97.79 107.95) (width 0.5588) (layer "B.Cu") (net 10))
 (segment (start 97.79 107.95) (end 94.14442 111.59558) (width 0.5588) (layer "B.Cu") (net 10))
 (segment (start 85.87442 111.59558) (end 84.52 112.95) (width 0.5588) (layer "B.Cu") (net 10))
 (segment (start 102.52 107.95) (end 102.52 117.95) (width 0.5588) (layer "B.Cu") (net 10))
 (segment (start 74.32 122.95) (end 69.32 117.95) (width 0.5588) (layer "B.Cu") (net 10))
 (segment (start 51.32 112.95) (end 51.32 122.95) (width 0.5588) (layer "B.Cu") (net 10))
 (segment (start 94.14442 111.59558) (end 85.87442 111.59558) (width 0.5588) (layer "B.Cu") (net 10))
 (segment (start 84.52 112.95) (end 84.52 122.95) (width 0.5588) (layer "B.Cu") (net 10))
 (segment (start 48.52 112.95) (end 48.52 122.95) (width 0.5588) (layer "B.Cu") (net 9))
 (segment (start 66.52 107.95) (end 52.35 107.95) (width 0.5588) (layer "B.Cu") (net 9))
 (segment (start 66.52 107.95) (end 66.52 117.95) (width 0.5588) (layer "B.Cu") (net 9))
 (segment (start 48.52 111.78) (end 50.8 109.5) (width 0.5588) (layer "B.Cu") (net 9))
 (segment (start 48.52 112.95) (end 48.52 111.78) (width 0.5588) (layer "B.Cu") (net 9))
 (segment (start 52.35 107.95) (end 50.8 109.5) (width 0.5588) (layer "B.Cu") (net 9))
 (segment (start 150.295428 116.404571) (end 97.971429 116.404571) (width 0.5588) (layer "F.Cu") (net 2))
 (segment (start 97.971429 116.404571) (end 95.123 119.253) (width 0.5588) (layer "F.Cu") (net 2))
 (segment (start 95.123 119.253) (end 95.123 122.345) (width 0.5588) (layer "F.Cu") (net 2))
 (segment (start 90.043 115.062) (end 90.043 122.345) (width 0.5588) (layer "F.Cu") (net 6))
 (segment (start 95.885 109.22) (end 90.043 115.062) (width 0.5588) (layer "F.Cu") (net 6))
 (segment (start 149.642285 109.22) (end 95.885 109.22) (width 0.5588) (layer "F.Cu") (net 6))
 (segment (start 150.295428 109.873143) (end 149.642285 109.22) (width 0.5588) (layer "F.Cu") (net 6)))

